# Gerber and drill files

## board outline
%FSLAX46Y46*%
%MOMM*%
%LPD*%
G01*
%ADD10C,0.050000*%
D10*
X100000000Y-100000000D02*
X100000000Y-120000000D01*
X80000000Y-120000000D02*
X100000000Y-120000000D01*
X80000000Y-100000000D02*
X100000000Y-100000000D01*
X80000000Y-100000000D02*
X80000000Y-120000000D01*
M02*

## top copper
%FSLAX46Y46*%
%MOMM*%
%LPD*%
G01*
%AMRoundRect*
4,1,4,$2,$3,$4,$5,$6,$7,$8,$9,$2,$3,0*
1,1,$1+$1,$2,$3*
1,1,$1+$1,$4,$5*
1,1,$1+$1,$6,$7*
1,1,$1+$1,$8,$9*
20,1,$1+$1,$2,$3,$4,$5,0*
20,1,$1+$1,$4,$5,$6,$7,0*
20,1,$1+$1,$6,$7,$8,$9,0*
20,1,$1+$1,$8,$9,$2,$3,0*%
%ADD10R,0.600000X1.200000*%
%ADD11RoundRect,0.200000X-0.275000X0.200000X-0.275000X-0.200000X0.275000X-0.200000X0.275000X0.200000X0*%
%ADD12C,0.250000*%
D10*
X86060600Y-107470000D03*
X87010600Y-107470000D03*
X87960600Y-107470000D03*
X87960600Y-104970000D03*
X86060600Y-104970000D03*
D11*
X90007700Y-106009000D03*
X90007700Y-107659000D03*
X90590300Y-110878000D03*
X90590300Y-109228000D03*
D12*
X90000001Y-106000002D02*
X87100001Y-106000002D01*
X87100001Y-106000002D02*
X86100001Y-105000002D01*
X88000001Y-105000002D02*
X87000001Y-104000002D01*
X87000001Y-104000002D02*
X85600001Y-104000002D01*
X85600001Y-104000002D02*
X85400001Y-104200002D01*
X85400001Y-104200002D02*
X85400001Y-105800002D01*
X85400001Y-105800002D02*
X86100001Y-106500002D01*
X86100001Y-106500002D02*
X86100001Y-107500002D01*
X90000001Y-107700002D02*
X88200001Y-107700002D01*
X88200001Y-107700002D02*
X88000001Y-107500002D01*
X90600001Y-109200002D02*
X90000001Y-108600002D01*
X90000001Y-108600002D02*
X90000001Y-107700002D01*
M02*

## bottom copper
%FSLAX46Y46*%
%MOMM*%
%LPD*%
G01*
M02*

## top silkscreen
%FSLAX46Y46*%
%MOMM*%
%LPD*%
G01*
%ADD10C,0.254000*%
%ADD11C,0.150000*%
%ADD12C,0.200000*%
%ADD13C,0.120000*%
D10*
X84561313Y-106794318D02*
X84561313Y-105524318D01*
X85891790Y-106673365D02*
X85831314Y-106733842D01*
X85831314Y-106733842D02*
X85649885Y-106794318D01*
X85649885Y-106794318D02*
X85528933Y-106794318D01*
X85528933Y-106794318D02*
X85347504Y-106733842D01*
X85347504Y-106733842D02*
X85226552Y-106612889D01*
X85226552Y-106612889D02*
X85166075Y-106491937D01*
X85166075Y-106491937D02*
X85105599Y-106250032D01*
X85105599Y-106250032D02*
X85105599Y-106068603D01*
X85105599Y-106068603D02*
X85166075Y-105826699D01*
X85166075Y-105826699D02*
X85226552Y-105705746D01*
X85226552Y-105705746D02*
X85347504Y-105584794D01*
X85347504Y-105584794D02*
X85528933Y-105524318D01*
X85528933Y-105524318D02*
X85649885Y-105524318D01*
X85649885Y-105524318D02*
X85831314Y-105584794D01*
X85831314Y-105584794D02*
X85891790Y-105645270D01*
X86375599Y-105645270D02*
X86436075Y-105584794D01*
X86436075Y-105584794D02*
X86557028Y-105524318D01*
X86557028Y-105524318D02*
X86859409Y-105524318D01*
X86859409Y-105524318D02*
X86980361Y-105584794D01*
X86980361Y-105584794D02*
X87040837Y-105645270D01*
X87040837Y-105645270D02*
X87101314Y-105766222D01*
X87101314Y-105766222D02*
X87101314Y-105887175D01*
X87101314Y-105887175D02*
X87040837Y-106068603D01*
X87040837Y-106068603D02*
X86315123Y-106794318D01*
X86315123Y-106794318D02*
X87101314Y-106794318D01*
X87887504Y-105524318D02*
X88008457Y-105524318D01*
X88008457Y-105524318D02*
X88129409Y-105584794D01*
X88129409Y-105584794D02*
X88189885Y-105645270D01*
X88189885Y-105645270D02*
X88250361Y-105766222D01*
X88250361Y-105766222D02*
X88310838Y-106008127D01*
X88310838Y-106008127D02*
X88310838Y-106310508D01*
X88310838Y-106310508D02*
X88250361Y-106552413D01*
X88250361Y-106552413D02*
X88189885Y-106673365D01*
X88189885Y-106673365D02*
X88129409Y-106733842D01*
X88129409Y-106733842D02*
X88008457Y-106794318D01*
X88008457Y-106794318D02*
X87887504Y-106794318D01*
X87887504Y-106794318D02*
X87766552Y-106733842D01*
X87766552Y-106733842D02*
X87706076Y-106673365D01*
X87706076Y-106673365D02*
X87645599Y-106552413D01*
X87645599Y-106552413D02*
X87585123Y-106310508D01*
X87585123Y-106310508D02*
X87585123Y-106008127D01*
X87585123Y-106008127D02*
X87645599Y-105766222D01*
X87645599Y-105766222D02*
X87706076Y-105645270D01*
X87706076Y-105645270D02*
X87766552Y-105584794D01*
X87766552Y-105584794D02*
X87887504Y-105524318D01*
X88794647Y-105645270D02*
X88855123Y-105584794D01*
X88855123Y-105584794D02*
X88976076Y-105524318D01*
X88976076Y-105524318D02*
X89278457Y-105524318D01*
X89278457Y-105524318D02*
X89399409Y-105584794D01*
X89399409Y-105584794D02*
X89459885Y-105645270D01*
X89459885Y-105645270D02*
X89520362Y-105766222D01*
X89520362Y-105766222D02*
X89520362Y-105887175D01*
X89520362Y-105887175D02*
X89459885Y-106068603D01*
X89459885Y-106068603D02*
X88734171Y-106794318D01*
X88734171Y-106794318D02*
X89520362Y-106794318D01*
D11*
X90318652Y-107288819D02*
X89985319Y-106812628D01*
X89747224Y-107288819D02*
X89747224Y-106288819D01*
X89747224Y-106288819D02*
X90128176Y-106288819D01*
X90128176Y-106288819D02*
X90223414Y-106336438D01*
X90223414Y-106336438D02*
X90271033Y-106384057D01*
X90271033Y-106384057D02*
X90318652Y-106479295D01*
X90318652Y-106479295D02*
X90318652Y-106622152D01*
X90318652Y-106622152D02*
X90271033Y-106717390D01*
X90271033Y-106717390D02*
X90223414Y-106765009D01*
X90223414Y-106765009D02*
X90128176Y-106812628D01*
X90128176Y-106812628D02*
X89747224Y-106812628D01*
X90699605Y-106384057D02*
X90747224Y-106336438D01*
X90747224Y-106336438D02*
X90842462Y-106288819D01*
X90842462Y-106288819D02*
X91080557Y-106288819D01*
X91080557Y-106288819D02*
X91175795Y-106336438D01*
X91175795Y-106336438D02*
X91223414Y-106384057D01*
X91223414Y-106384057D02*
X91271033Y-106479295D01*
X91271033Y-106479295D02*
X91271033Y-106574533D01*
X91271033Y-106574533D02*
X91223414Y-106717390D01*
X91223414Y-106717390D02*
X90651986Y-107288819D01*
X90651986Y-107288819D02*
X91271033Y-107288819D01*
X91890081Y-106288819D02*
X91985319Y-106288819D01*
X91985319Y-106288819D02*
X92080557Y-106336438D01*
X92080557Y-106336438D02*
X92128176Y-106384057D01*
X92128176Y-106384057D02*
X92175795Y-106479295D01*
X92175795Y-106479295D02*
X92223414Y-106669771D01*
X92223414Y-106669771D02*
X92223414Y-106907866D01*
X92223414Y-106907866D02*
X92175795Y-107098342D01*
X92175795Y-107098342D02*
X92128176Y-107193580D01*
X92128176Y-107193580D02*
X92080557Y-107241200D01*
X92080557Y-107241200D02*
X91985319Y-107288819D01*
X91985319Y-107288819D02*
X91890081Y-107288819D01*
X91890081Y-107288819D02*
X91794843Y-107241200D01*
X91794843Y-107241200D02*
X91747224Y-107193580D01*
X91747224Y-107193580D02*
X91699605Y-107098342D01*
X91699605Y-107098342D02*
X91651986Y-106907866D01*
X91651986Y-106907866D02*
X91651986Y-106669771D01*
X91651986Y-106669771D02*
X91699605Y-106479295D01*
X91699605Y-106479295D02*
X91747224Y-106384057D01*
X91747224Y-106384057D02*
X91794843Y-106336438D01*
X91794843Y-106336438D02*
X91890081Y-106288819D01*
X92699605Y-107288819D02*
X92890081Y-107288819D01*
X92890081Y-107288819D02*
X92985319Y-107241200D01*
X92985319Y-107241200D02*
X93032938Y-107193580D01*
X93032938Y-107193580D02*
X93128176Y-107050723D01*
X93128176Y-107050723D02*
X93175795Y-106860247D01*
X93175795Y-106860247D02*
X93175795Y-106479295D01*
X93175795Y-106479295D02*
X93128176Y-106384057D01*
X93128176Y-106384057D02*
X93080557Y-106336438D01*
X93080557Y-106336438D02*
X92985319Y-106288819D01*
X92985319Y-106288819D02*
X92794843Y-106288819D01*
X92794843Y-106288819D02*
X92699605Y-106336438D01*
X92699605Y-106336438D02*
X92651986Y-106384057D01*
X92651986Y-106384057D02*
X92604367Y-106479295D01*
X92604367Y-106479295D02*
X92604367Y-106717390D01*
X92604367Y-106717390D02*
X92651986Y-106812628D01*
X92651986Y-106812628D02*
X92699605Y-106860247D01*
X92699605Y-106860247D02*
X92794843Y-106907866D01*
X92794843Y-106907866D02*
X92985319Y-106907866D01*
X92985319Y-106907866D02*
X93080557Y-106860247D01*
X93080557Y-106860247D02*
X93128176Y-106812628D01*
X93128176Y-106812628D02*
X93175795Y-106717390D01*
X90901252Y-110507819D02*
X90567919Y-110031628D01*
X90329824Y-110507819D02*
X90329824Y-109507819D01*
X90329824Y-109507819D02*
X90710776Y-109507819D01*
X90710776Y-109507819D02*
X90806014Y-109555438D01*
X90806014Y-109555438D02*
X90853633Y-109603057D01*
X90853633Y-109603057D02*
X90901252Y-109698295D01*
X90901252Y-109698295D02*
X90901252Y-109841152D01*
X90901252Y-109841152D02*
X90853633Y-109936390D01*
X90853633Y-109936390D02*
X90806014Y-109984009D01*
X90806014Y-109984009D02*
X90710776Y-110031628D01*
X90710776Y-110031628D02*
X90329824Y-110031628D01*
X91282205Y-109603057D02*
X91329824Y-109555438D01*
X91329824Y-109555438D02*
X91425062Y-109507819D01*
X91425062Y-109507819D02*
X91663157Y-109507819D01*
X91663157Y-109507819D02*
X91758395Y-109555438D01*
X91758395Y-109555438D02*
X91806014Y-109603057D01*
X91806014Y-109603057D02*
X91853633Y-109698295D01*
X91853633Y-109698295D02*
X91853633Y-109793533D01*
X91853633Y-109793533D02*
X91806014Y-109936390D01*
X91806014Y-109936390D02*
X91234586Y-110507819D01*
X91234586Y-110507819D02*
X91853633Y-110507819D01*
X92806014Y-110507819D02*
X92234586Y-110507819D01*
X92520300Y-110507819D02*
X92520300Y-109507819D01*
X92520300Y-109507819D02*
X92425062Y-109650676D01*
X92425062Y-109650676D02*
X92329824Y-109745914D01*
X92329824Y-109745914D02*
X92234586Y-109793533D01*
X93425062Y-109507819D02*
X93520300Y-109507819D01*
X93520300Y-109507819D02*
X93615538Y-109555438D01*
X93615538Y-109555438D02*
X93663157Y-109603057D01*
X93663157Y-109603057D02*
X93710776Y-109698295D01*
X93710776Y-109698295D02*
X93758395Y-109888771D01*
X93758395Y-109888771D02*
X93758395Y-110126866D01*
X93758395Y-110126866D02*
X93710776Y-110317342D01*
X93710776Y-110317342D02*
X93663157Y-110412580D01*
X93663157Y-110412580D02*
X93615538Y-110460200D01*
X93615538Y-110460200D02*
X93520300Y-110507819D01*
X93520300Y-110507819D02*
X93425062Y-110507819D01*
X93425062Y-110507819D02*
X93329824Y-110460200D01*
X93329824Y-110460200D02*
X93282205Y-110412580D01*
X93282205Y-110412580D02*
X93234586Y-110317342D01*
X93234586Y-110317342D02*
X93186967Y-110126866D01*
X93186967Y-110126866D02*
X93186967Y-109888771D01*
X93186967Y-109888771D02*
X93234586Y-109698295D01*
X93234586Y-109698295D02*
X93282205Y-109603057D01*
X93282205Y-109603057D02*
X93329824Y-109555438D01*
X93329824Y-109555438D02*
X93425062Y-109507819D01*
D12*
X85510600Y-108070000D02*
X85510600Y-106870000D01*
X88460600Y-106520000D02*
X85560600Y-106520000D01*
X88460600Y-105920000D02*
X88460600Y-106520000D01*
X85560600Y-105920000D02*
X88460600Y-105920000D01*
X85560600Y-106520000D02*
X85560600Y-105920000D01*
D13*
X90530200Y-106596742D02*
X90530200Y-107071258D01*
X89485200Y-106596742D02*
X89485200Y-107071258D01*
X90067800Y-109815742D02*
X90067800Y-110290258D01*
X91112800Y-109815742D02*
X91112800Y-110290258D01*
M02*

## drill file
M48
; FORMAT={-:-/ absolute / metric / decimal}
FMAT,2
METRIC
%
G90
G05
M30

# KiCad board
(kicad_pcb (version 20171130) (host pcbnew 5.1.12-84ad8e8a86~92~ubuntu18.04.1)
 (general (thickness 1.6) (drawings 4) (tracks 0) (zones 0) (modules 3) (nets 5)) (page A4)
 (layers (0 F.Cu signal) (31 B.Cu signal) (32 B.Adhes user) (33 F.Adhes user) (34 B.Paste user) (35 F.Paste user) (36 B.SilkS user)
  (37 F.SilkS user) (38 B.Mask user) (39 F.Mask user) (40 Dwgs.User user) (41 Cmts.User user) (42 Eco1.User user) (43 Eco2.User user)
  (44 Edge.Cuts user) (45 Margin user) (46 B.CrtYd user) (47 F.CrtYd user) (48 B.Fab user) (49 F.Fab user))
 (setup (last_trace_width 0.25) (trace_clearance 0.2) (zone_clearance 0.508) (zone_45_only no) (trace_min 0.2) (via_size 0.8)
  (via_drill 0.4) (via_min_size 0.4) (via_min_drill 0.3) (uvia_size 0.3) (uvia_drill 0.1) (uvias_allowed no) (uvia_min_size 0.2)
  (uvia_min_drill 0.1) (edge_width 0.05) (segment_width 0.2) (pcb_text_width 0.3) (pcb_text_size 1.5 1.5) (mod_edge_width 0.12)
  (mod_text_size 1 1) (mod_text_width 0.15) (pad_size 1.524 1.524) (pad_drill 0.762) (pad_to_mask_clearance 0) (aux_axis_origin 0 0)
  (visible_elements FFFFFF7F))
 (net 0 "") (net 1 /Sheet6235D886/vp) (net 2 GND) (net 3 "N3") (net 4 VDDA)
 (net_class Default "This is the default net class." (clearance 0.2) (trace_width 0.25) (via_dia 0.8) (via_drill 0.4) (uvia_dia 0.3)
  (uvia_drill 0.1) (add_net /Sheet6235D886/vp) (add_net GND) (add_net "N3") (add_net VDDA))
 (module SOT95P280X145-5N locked (layer F.Cu) (at 87.010600 106.220000 90.000000)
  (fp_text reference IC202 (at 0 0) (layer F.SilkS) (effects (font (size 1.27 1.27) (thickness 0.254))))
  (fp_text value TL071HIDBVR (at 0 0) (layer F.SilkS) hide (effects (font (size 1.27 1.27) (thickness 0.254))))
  (fp_line (start -1.85 -1.5) (end -0.65 -1.5) (layer F.SilkS) (width 0.2))
  (fp_line (start -0.3 1.45) (end -0.3 -1.45) (layer F.SilkS) (width 0.2))
  (fp_line (start 0.3 1.45) (end -0.3 1.45) (layer F.SilkS) (width 0.2))
  (fp_line (start 0.3 -1.45) (end 0.3 1.45) (layer F.SilkS) (width 0.2))
  (fp_line (start -0.3 -1.45) (end 0.3 -1.45) (layer F.SilkS) (width 0.2))
  (pad 1 smd rect (at -1.25 -0.95 180.000000) (size 0.6 1.2) (layers F.Cu F.Mask F.Paste) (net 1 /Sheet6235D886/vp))
  (pad 2 smd rect (at -1.25 0 180.000000) (size 0.6 1.2) (layers F.Cu F.Mask F.Paste) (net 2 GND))
  (pad 3 smd rect (at -1.25 0.95 180.000000) (size 0.6 1.2) (layers F.Cu F.Mask F.Paste) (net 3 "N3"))
  (pad 4 smd rect (at 1.25 0.95 180.000000) (size 0.6 1.2) (layers F.Cu F.Mask F.Paste) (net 1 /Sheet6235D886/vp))
  (pad 5 smd rect (at 1.25 -0.95 180.000000) (size 0.6 1.2) (layers F.Cu F.Mask F.Paste) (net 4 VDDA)))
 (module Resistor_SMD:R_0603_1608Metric (layer F.Cu) (at 90.007700 106.834000 270.000000)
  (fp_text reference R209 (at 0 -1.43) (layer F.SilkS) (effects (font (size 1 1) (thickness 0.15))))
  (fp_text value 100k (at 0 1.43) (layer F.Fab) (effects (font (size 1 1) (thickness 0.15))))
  (fp_line (start -0.237258 -0.5225) (end 0.237258 -0.5225) (layer F.SilkS) (width 0.12))
  (fp_line (start -0.237258 0.5225) (end 0.237258 0.5225) (layer F.SilkS) (width 0.12))
  (pad 1 smd roundrect (at -0.825 0 270.000000) (size 0.8 0.95) (layers F.Cu F.Mask F.Paste) (roundrect_rratio 0.25) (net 4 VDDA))
  (pad 2 smd roundrect (at 0.825 0 270.000000) (size 0.8 0.95) (layers F.Cu F.Mask F.Paste) (roundrect_rratio 0.25) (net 3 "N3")))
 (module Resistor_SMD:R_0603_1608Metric (layer F.Cu) (at 90.590300 110.053000 270.000000)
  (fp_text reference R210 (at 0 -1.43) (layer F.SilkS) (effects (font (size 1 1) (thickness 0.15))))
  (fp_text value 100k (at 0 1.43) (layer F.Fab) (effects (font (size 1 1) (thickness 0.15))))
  (fp_line (start -0.237258 0.5225) (end 0.237258 0.5225) (layer F.SilkS) (width 0.12))
  (fp_line (start -0.237258 -0.5225) (end 0.237258 -0.5225) (layer F.SilkS) (width 0.12))
  (pad 2 smd roundrect (at 0.825 0 270.000000) (size 0.8 0.95) (layers F.Cu F.Mask F.Paste) (roundrect_rratio 0.25) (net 2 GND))
  (pad 1 smd roundrect (at -0.825 0 270.000000) (size 0.8 0.95) (layers F.Cu F.Mask F.Paste) (roundrect_rratio 0.25) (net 3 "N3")))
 (gr_line (start 100 100) (end 100 120) (layer Edge.Cuts) (width 0.05))
 (gr_line (start 80 120) (end 100 120) (layer Edge.Cuts) (width 0.05))
 (gr_line (start 80 100) (end 100 100) (layer Edge.Cuts) (width 0.05))
 (gr_line (start 80 100) (end 80 120) (layer Edge.Cuts) (width 0.05))
 (segment (start 90.000001 106.000002) (end 87.100001 106.000002) (width 0.250000) (layer F.Cu) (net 4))
 (segment (start 87.100001 106.000002) (end 86.100001 105.000002) (width 0.250000) (layer F.Cu) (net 4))
 (segment (start 88.000001 105.000002) (end 87.000001 104.000002) (width 0.250000) (layer F.Cu) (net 1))
 (segment (start 87.000001 104.000002) (end 85.600001 104.000002) (width 0.250000) (layer F.Cu) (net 1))
 (segment (start 85.600001 104.000002) (end 85.400001 104.200002) (width 0.250000) (layer F.Cu) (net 1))
 (segment (start 85.400001 104.200002) (end 85.400001 105.800002) (width 0.250000) (layer F.Cu) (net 1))
 (segment (start 85.400001 105.800002) (end 86.100001 106.500002) (width 0.250000) (layer F.Cu) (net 1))
 (segment (start 86.100001 106.500002) (end 86.100001 107.500002) (width 0.250000) (layer F.Cu) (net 1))
 (segment (start 90.000001 107.700002) (end 88.200001 107.700002) (width 0.250000) (layer F.Cu) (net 3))
 (segment (start 88.200001 107.700002) (end 88.000001 107.500002) (width 0.250000) (layer F.Cu) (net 3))
 (segment (start 90.600001 109.200002) (end 90.000001 108.600002) (width 0.250000) (layer F.Cu) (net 3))
 (segment (start 90.000001 108.600002) (end 90.000001 107.700002) (width 0.250000) (layer F.Cu) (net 3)))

